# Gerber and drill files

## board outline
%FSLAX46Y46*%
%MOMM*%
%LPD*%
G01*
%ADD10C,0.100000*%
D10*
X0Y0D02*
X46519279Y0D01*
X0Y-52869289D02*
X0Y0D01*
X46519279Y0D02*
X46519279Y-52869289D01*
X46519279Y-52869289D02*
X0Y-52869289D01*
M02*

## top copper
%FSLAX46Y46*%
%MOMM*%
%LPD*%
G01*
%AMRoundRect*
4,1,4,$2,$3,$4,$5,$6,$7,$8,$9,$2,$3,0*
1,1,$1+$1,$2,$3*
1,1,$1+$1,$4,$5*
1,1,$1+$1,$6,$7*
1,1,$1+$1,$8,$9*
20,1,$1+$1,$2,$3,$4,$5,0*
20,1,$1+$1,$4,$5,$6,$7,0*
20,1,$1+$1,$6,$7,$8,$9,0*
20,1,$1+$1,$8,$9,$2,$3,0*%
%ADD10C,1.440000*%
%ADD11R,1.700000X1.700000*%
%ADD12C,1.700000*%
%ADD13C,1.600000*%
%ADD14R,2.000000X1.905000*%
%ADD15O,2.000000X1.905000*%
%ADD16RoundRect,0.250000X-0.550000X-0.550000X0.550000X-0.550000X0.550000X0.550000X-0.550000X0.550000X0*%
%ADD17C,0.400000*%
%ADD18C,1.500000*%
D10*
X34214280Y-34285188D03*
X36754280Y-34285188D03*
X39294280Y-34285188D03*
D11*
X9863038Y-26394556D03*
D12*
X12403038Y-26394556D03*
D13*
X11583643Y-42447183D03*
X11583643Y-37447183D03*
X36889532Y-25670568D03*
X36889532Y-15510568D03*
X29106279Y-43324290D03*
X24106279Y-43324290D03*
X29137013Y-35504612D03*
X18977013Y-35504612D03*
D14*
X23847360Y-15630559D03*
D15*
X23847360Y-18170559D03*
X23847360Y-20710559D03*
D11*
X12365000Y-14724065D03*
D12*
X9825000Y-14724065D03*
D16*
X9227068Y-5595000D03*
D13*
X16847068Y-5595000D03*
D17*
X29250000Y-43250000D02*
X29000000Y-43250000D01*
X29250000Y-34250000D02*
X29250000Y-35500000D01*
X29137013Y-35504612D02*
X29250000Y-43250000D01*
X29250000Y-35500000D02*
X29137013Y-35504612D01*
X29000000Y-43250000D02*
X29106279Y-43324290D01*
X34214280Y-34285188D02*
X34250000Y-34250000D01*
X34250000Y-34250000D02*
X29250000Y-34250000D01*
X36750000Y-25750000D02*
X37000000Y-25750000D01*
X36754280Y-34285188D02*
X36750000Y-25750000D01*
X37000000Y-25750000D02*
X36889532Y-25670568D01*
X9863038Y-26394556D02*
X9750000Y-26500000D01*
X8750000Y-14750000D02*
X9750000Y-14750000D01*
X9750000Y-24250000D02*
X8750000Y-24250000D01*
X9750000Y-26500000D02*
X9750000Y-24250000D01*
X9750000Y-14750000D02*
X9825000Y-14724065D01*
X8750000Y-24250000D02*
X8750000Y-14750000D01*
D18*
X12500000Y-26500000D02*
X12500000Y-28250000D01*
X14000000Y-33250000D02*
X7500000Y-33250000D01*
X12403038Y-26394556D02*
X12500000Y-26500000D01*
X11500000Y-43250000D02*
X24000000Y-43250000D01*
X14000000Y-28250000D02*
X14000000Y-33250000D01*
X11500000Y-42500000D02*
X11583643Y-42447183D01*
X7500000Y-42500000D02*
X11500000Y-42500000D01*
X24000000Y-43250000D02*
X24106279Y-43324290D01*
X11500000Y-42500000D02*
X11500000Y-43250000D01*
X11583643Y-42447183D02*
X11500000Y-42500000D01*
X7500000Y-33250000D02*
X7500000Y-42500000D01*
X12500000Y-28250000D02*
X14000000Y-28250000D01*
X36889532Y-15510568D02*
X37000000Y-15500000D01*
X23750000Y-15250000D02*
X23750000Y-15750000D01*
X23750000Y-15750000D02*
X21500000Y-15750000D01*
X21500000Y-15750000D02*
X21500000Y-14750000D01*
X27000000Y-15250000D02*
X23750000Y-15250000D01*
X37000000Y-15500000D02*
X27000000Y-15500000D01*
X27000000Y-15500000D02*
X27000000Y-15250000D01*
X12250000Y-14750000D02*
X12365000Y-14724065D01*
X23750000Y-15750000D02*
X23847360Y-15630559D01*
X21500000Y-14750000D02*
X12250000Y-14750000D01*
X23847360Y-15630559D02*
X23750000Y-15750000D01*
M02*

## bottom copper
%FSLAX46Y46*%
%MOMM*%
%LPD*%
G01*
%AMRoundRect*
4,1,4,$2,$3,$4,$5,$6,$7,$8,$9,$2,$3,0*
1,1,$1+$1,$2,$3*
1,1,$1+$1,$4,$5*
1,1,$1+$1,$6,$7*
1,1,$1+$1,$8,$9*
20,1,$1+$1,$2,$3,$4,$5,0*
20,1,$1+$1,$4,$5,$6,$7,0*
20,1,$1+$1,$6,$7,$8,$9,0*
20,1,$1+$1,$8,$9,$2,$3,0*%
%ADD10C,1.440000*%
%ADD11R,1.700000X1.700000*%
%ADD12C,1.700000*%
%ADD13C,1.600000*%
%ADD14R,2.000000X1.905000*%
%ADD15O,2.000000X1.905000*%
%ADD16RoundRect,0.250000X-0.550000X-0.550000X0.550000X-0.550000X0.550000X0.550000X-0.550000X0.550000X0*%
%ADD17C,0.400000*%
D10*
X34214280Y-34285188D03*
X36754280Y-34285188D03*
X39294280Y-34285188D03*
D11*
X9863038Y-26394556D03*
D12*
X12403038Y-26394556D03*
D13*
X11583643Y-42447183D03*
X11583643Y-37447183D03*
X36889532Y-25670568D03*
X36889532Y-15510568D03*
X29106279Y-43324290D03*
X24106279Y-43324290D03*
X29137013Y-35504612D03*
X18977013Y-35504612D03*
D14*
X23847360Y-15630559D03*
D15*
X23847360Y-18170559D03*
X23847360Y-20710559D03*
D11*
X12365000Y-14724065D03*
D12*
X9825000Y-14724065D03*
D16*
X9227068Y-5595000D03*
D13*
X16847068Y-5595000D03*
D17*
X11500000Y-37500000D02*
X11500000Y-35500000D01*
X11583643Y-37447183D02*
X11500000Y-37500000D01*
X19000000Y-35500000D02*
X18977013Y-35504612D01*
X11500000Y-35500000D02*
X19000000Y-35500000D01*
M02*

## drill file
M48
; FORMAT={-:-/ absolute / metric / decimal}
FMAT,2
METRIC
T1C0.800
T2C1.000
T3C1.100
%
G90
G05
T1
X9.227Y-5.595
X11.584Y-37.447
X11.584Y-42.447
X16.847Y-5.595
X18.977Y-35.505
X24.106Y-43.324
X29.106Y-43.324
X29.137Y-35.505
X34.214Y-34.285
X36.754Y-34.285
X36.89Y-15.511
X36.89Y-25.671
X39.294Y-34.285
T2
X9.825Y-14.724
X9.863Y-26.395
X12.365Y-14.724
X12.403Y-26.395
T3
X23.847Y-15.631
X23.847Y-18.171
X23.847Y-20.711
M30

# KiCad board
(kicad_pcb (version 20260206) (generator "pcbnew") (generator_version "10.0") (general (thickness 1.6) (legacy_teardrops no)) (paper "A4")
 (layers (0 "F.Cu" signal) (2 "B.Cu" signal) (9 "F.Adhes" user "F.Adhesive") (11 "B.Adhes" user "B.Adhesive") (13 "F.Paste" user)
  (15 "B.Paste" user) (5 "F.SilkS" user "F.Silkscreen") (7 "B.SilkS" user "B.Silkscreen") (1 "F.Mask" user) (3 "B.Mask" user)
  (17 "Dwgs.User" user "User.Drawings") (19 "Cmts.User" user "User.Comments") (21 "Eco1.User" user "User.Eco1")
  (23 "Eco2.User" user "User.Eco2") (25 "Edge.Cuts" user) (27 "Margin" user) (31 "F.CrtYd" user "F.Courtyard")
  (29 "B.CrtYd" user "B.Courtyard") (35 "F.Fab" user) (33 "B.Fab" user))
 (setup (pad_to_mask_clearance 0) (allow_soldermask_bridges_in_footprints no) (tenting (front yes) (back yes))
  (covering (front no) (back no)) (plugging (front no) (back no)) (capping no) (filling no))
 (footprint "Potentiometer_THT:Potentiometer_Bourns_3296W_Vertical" (layer "F.Cu") (at 34.21428 34.285188 180)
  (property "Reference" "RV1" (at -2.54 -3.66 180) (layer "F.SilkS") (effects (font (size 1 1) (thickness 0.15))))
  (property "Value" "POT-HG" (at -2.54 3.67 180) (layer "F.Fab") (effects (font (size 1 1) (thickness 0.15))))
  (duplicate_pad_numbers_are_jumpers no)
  (pad "1" thru_hole circle (at 0 0 180) (size 1.44 1.44) (drill 0.8) (layers "*.Cu" "*.Mask") (remove_unused_layers no) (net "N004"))
  (pad "2" thru_hole circle (at -2.54 0 180) (size 1.44 1.44) (drill 0.8) (layers "*.Cu" "*.Mask") (remove_unused_layers no) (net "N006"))
  (pad "3" thru_hole circle (at -5.08 0 180) (size 1.44 1.44) (drill 0.8) (layers "*.Cu" "*.Mask") (remove_unused_layers no)))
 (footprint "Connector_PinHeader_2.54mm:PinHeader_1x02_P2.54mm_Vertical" (layer "F.Cu") (at 9.863038 26.394556 90)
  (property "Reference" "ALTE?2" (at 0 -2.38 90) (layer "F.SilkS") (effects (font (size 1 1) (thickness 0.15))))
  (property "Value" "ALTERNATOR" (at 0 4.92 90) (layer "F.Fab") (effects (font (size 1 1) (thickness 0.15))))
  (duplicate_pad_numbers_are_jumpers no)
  (pad "1" thru_hole rect (at 0 0 90) (size 1.7 1.7) (drill 1) (layers "*.Cu" "*.Mask") (remove_unused_layers no) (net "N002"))
  (pad "2" thru_hole circle (at 0 2.54 90) (size 1.7 1.7) (drill 1) (layers "*.Cu" "*.Mask") (remove_unused_layers no) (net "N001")))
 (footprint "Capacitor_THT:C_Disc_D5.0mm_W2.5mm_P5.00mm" (layer "F.Cu") (at 11.583643 42.447183 90)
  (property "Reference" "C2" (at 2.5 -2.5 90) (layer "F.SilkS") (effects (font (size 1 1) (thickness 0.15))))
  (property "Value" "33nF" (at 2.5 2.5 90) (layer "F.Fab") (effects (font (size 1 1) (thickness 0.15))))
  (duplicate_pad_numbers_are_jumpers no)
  (pad "1" thru_hole circle (at 0 0 90) (size 1.6 1.6) (drill 0.8) (layers "*.Cu" "*.Mask") (remove_unused_layers no) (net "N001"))
  (pad "2" thru_hole circle (at 5 0 90) (size 1.6 1.6) (drill 0.8) (layers "*.Cu" "*.Mask") (remove_unused_layers no) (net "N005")))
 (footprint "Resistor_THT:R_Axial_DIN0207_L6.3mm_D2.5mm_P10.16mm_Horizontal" (layer "F.Cu") (at 36.889532 25.670568 90)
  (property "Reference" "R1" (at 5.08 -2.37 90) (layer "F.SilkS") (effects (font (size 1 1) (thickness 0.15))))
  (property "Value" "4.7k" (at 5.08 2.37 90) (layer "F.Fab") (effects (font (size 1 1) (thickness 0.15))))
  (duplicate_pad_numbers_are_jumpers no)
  (pad "1" thru_hole circle (at 0 0 90) (size 1.6 1.6) (drill 0.8) (layers "*.Cu" "*.Mask") (remove_unused_layers no) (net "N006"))
  (pad "2" thru_hole circle (at 10.16 0 90) (size 1.6 1.6) (drill 0.8) (layers "*.Cu" "*.Mask") (remove_unused_layers no) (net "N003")))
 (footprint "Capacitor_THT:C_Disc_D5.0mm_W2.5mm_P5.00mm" (layer "F.Cu") (at 29.106279 43.32429 180)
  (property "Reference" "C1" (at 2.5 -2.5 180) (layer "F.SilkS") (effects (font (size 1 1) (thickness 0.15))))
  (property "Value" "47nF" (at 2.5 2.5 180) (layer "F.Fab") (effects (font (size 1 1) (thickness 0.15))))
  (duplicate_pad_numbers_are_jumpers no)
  (pad "1" thru_hole circle (at 0 0 180) (size 1.6 1.6) (drill 0.8) (layers "*.Cu" "*.Mask") (remove_unused_layers no) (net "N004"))
  (pad "2" thru_hole circle (at 5 0 180) (size 1.6 1.6) (drill 0.8) (layers "*.Cu" "*.Mask") (remove_unused_layers no) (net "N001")))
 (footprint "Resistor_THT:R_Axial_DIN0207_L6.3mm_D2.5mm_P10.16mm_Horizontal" (layer "F.Cu") (at 29.137013 35.504612 180)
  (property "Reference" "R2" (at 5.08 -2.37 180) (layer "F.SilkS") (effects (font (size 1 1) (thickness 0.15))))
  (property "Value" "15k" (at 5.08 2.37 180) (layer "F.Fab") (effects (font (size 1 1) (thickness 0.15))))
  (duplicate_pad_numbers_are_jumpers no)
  (pad "1" thru_hole circle (at 0 0 180) (size 1.6 1.6) (drill 0.8) (layers "*.Cu" "*.Mask") (remove_unused_layers no) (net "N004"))
  (pad "2" thru_hole circle (at 10.16 0 180) (size 1.6 1.6) (drill 0.8) (layers "*.Cu" "*.Mask") (remove_unused_layers no) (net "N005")))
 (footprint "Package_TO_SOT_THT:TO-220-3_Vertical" (layer "F.Cu") (at 23.84736 15.630559 -90)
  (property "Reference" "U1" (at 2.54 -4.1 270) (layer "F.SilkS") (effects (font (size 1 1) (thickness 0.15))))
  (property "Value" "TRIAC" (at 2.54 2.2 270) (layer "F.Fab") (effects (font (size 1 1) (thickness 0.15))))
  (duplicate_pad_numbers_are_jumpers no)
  (pad "1" thru_hole rect (at 0 0 270) (size 1.905 2) (drill 1.1) (layers "*.Cu" "*.Mask") (remove_unused_layers no) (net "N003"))
  (pad "2" thru_hole oval (at 2.54 0 270) (size 1.905 2) (drill 1.1) (layers "*.Cu" "*.Mask") (remove_unused_layers no) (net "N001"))
  (pad "3" thru_hole oval (at 5.08 0 270) (size 1.905 2) (drill 1.1) (layers "*.Cu" "*.Mask") (remove_unused_layers no) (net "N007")))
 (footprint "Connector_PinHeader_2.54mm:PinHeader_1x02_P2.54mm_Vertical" (layer "F.Cu") (at 12.365 14.724065 -90)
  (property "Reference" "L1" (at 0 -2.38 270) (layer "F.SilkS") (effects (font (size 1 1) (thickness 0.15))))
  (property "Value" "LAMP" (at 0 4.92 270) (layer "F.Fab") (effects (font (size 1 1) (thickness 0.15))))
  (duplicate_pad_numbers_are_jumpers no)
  (pad "1" thru_hole rect (at 0 0 270) (size 1.7 1.7) (drill 1) (layers "*.Cu" "*.Mask") (remove_unused_layers no) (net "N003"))
  (pad "2" thru_hole circle (at 0 2.54 270) (size 1.7 1.7) (drill 1) (layers "*.Cu" "*.Mask") (remove_unused_layers no) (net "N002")))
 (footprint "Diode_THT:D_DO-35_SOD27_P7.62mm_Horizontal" (layer "F.Cu") (at 9.227068 5.595)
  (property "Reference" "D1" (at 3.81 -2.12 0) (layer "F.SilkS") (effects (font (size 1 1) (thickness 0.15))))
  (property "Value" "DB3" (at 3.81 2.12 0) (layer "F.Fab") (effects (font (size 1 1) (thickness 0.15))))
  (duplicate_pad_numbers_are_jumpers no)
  (pad "1" thru_hole roundrect (at 0 0) (size 1.6 1.6) (drill 0.8) (layers "*.Cu" "*.Mask") (remove_unused_layers no)
   (roundrect_rratio 0.15625))
  (pad "2" thru_hole circle (at 7.62 0) (size 1.6 1.6) (drill 0.8) (layers "*.Cu" "*.Mask") (remove_unused_layers no)))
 (gr_line (start 0 0) (end 46.519279 0) (stroke (width 0.1) (type default)) (layer "Edge.Cuts"))
 (gr_line (start 0 52.869289) (end 0 0) (stroke (width 0.1) (type default)) (layer "Edge.Cuts"))
 (gr_line (start 46.519279 0) (end 46.519279 52.869289) (stroke (width 0.1) (type default)) (layer "Edge.Cuts"))
 (gr_line (start 46.519279 52.869289) (end 0 52.869289) (stroke (width 0.1) (type default)) (layer "Edge.Cuts"))
 (segment (start 29.25 43.25) (end 29 43.25) (width 0.4) (layer "F.Cu") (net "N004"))
 (segment (start 29.25 34.25) (end 29.25 35.5) (width 0.4) (layer "F.Cu") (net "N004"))
 (segment (start 29.137013 35.504612) (end 29.25 43.25) (width 0.4) (layer "F.Cu") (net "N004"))
 (segment (start 29.25 35.5) (end 29.137013 35.504612) (width 0.4) (layer "F.Cu") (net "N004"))
 (segment (start 29 43.25) (end 29.106279 43.32429) (width 0.4) (layer "F.Cu") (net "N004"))
 (segment (start 34.21428 34.285188) (end 34.25 34.25) (width 0.4) (layer "F.Cu") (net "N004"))
 (segment (start 34.25 34.25) (end 29.25 34.25) (width 0.4) (layer "F.Cu") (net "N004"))
 (segment (start 36.75 25.75) (end 37 25.75) (width 0.4) (layer "F.Cu") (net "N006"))
 (segment (start 36.75428 34.285188) (end 36.75 25.75) (width 0.4) (layer "F.Cu") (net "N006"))
 (segment (start 37 25.75) (end 36.889532 25.670568) (width 0.4) (layer "F.Cu") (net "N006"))
 (segment (start 9.863038 26.394556) (end 9.75 26.5) (width 0.4) (layer "F.Cu") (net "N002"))
 (segment (start 8.75 14.75) (end 9.75 14.75) (width 0.4) (layer "F.Cu") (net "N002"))
 (segment (start 9.75 24.25) (end 8.75 24.25) (width 0.4) (layer "F.Cu") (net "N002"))
 (segment (start 9.75 26.5) (end 9.75 24.25) (width 0.4) (layer "F.Cu") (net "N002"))
 (segment (start 9.75 14.75) (end 9.825 14.724065) (width 0.4) (layer "F.Cu") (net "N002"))
 (segment (start 8.75 24.25) (end 8.75 14.75) (width 0.4) (layer "F.Cu") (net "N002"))
 (segment (start 12.5 26.5) (end 12.5 28.25) (width 1.5) (layer "F.Cu") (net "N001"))
 (segment (start 14 33.25) (end 7.5 33.25) (width 1.5) (layer "F.Cu") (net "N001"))
 (segment (start 12.403038 26.394556) (end 12.5 26.5) (width 1.5) (layer "F.Cu") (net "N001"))
 (segment (start 11.5 43.25) (end 24 43.25) (width 1.5) (layer "F.Cu") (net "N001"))
 (segment (start 14 28.25) (end 14 33.25) (width 1.5) (layer "F.Cu") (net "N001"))
 (segment (start 11.5 42.5) (end 11.583643 42.447183) (width 1.5) (layer "F.Cu") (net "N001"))
 (segment (start 7.5 42.5) (end 11.5 42.5) (width 1.5) (layer "F.Cu") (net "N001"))
 (segment (start 24 43.25) (end 24.106279 43.32429) (width 1.5) (layer "F.Cu") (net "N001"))
 (segment (start 11.5 42.5) (end 11.5 43.25) (width 1.5) (layer "F.Cu") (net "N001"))
 (segment (start 11.583643 42.447183) (end 11.5 42.5) (width 1.5) (layer "F.Cu") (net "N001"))
 (segment (start 7.5 33.25) (end 7.5 42.5) (width 1.5) (layer "F.Cu") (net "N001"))
 (segment (start 12.5 28.25) (end 14 28.25) (width 1.5) (layer "F.Cu") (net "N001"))
 (segment (start 11.5 37.5) (end 11.5 35.5) (width 0.4) (layer "B.Cu") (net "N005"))
 (segment (start 11.583643 37.447183) (end 11.5 37.5) (width 0.4) (layer "B.Cu") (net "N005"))
 (segment (start 19 35.5) (end 18.977013 35.504612) (width 0.4) (layer "B.Cu") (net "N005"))
 (segment (start 11.5 35.5) (end 19 35.5) (width 0.4) (layer "B.Cu") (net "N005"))
 (segment (start 36.889532 15.510568) (end 37 15.5) (width 1.5) (layer "F.Cu") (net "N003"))
 (segment (start 23.75 15.25) (end 23.75 15.75) (width 1.5) (layer "F.Cu") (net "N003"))
 (segment (start 23.75 15.75) (end 21.5 15.75) (width 1.5) (layer "F.Cu") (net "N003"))
 (segment (start 21.5 15.75) (end 21.5 14.75) (width 1.5) (layer "F.Cu") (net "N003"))
 (segment (start 27 15.25) (end 23.75 15.25) (width 1.5) (layer "F.Cu") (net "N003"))
 (segment (start 37 15.5) (end 27 15.5) (width 1.5) (layer "F.Cu") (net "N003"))
 (segment (start 27 15.5) (end 27 15.25) (width 1.5) (layer "F.Cu") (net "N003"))
 (segment (start 12.25 14.75) (end 12.365 14.724065) (width 1.5) (layer "F.Cu") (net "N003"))
 (segment (start 23.75 15.75) (end 23.84736 15.630559) (width 1.5) (layer "F.Cu") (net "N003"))
 (segment (start 21.5 14.75) (end 12.25 14.75) (width 1.5) (layer "F.Cu") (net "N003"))
 (segment (start 23.84736 15.630559) (end 23.75 15.75) (width 1.5) (layer "F.Cu") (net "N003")))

